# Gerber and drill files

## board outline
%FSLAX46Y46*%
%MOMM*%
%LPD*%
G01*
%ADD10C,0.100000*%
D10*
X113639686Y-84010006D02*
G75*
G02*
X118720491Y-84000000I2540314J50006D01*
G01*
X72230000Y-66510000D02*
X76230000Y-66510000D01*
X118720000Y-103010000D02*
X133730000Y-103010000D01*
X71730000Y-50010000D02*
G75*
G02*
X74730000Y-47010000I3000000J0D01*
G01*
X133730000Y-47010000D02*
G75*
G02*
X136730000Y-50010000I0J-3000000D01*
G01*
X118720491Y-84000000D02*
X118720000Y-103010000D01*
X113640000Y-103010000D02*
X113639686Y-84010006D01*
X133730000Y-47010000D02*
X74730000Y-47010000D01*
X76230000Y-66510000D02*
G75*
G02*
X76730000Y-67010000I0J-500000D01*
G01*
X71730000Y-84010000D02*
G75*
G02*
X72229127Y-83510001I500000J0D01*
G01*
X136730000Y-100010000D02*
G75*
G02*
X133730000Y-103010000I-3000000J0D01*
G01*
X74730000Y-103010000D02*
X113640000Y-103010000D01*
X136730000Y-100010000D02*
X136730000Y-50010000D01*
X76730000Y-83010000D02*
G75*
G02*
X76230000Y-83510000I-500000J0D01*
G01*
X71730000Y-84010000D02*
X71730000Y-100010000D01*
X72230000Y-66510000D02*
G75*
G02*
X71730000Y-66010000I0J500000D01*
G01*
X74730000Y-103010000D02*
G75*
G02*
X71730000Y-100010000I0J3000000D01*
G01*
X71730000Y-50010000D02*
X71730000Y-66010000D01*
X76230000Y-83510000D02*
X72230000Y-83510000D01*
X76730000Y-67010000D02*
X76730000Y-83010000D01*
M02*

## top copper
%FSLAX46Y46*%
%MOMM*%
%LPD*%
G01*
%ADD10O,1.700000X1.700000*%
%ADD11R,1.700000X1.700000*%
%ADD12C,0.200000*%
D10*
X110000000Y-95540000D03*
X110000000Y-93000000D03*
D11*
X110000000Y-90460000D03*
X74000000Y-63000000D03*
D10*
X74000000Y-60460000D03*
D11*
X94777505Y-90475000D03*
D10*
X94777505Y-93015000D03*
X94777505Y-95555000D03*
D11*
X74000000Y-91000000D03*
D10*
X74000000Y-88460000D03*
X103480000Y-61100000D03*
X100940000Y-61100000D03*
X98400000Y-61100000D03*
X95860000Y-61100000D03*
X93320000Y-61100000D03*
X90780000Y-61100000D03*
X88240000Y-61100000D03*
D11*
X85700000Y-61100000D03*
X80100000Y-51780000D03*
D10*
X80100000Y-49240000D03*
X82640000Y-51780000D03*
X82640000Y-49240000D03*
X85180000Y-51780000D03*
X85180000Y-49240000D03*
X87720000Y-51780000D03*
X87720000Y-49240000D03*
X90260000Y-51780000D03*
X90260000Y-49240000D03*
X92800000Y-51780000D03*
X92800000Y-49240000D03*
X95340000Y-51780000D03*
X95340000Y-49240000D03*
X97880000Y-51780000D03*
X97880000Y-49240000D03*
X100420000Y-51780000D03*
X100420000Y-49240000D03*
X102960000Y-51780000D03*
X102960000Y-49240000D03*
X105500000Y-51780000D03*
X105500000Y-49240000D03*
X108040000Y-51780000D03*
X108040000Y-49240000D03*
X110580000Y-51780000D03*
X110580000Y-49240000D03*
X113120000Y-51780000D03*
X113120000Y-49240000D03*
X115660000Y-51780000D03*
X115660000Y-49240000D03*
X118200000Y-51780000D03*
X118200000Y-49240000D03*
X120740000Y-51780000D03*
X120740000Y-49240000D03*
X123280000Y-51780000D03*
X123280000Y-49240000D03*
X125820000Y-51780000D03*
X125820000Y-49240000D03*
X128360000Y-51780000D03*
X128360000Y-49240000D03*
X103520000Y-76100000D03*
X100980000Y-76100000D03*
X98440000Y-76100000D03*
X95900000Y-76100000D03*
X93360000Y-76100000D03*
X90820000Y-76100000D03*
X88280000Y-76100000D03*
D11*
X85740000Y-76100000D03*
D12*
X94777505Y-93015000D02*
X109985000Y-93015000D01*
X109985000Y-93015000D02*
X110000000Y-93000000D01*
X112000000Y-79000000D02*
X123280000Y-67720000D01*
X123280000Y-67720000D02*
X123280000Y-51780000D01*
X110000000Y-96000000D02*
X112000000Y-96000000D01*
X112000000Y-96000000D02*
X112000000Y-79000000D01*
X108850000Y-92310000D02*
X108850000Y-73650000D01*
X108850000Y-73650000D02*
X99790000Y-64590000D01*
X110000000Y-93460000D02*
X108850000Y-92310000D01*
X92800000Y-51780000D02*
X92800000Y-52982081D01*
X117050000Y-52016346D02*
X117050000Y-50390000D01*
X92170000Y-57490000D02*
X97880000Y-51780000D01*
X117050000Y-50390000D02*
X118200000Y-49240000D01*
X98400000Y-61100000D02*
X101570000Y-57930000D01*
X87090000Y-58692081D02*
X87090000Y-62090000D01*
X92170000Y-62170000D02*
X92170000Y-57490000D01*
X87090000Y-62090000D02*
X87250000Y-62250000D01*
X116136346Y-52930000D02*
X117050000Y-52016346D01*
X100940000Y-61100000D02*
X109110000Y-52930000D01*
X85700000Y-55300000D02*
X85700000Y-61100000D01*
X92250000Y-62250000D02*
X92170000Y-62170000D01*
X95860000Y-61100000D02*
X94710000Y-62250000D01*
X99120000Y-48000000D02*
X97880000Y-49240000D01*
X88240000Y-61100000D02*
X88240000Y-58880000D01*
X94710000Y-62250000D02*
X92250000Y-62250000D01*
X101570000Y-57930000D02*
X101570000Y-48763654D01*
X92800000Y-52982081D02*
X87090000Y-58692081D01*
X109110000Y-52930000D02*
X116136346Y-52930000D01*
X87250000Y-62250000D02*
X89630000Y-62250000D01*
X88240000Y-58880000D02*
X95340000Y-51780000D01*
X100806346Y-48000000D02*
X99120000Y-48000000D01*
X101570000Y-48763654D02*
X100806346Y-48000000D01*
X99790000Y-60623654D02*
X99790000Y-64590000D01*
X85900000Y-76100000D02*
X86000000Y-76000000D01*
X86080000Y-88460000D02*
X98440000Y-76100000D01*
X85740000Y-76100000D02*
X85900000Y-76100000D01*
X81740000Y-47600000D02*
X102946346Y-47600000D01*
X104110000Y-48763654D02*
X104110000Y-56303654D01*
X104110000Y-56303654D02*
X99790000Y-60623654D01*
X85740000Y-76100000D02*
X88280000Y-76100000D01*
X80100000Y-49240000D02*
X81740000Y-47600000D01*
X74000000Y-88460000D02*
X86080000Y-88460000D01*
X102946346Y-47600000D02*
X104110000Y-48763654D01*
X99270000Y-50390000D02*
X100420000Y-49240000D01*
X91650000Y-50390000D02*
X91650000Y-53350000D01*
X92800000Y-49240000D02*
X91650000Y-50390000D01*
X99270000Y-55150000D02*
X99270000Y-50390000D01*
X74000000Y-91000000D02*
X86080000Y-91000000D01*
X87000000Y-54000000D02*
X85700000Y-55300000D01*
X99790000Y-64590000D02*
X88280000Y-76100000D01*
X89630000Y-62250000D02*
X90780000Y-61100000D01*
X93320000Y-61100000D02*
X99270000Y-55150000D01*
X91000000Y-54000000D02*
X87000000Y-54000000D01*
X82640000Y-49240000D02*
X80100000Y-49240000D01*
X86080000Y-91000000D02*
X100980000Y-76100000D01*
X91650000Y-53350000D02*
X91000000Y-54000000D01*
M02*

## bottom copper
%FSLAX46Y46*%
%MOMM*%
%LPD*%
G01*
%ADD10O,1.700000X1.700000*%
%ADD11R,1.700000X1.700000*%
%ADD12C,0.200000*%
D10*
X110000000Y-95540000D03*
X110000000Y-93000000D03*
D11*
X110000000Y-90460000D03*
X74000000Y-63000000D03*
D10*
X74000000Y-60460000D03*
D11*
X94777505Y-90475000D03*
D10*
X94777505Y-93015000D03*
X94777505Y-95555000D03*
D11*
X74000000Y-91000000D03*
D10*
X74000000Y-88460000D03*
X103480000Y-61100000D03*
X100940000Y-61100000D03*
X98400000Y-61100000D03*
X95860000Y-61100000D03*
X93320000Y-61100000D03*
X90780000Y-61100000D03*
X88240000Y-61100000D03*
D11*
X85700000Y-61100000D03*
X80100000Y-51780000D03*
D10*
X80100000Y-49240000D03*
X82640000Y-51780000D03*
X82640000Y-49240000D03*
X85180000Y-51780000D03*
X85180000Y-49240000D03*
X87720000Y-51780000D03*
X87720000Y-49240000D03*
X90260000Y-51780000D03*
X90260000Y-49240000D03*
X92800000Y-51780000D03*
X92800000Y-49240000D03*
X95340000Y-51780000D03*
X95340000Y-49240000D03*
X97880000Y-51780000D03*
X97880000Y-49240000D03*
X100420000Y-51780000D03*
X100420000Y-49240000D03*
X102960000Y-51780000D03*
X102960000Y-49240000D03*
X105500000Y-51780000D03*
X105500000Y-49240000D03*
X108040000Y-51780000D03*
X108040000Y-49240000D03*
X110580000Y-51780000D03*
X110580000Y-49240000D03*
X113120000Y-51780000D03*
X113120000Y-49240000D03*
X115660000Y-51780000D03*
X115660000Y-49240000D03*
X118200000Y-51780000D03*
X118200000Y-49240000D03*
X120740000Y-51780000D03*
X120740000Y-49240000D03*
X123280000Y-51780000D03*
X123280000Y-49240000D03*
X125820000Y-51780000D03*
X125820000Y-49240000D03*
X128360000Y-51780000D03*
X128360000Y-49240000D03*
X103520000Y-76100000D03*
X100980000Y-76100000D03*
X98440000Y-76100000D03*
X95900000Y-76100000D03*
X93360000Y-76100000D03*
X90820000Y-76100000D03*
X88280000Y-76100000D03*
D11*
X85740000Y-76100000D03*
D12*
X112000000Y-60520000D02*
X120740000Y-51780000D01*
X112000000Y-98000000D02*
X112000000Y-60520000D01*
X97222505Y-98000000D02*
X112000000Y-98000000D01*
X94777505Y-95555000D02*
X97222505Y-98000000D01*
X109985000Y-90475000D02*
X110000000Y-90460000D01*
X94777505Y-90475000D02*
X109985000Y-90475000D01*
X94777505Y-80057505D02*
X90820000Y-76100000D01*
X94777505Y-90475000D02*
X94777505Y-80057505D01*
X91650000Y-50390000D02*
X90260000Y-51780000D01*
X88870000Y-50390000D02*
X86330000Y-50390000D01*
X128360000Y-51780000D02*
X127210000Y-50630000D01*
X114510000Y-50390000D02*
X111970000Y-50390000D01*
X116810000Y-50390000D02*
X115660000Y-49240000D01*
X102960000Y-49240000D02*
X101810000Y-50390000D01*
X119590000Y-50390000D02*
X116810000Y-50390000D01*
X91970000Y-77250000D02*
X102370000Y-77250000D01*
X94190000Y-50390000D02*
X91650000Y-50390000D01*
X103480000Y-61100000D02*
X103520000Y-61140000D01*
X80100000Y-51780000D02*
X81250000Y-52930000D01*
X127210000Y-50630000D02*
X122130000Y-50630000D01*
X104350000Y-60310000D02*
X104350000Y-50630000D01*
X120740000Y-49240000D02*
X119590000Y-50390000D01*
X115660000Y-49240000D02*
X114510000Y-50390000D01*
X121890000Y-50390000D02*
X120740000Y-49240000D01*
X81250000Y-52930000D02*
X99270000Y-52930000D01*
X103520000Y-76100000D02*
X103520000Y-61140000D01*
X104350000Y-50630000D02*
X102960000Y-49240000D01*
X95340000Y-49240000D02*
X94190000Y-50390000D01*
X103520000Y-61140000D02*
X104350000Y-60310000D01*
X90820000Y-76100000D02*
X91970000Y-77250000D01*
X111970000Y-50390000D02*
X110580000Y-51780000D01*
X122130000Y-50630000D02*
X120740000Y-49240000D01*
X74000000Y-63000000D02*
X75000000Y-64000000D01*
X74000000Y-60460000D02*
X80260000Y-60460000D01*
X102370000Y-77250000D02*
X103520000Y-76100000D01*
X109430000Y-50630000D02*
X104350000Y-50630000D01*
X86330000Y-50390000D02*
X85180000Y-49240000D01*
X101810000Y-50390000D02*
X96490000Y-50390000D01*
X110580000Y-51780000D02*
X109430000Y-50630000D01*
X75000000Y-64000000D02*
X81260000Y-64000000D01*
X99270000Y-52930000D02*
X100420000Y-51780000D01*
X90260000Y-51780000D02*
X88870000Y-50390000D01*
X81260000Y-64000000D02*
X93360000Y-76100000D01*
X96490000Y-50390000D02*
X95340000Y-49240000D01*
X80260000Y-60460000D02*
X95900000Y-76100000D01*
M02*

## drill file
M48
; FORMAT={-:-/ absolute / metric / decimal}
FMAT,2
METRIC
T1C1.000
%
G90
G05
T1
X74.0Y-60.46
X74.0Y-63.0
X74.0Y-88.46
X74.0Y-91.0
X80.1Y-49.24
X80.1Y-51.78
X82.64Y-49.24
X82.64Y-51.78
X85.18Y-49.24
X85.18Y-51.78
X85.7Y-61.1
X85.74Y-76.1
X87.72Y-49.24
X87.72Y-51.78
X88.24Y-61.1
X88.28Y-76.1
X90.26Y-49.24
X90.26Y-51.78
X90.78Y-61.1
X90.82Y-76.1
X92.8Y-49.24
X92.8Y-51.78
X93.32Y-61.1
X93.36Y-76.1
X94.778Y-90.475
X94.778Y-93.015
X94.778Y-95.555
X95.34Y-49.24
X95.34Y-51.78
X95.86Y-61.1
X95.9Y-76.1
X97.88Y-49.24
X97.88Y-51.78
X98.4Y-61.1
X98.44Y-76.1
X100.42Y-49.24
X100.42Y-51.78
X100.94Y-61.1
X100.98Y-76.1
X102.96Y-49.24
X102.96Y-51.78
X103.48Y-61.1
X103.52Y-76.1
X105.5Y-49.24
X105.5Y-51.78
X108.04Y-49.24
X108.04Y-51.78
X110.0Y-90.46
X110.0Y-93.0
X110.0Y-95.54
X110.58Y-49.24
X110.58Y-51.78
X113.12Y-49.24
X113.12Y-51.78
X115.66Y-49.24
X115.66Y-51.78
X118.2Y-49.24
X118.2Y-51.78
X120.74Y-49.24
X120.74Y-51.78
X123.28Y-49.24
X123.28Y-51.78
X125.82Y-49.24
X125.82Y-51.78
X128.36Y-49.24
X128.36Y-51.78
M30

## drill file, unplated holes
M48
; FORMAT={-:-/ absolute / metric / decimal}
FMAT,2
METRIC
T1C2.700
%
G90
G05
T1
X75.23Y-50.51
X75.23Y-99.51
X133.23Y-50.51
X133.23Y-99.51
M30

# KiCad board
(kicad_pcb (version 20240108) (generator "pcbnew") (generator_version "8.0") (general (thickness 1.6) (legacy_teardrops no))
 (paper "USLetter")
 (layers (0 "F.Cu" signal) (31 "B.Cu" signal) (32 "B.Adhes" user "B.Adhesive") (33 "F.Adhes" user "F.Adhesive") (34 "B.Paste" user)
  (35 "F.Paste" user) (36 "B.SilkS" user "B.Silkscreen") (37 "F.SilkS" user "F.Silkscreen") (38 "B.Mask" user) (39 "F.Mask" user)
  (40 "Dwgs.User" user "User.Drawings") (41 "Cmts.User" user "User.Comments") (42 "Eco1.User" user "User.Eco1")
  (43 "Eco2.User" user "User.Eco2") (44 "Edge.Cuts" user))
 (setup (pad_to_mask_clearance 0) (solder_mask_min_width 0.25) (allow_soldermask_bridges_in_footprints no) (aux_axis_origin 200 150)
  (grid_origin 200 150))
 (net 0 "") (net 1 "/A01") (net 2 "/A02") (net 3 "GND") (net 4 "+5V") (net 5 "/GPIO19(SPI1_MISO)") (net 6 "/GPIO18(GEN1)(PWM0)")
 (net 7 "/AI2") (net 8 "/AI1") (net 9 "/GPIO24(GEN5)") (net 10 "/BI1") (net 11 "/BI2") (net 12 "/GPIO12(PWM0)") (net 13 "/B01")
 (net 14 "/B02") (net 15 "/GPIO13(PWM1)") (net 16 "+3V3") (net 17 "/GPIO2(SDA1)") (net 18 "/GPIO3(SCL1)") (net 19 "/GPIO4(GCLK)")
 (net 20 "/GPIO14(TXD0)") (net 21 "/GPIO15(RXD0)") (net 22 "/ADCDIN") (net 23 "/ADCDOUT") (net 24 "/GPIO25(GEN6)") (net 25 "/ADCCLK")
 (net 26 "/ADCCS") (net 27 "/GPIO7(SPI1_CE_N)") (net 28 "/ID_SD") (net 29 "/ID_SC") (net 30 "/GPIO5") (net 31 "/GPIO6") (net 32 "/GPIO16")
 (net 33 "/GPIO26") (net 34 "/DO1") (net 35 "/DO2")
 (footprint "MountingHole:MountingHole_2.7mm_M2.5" (layer "F.Cu") (at 133.23 99.51)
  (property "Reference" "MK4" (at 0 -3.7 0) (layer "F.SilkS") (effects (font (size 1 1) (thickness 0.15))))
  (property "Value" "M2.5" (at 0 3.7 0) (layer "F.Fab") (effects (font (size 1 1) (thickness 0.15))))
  (pad "" np_thru_hole circle (at 0 0) (size 2.7 2.7) (drill 2.7) (layers "*.Cu" "*.Mask")))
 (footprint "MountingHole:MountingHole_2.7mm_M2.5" (layer "F.Cu") (at 75.23 99.51)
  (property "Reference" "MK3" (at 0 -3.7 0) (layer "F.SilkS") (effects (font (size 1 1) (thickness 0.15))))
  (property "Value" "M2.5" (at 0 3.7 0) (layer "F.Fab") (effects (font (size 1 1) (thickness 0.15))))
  (pad "" np_thru_hole circle (at 0 0) (size 2.7 2.7) (drill 2.7) (layers "*.Cu" "*.Mask")))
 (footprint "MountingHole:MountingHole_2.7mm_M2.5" (layer "F.Cu") (at 75.23 50.51 180)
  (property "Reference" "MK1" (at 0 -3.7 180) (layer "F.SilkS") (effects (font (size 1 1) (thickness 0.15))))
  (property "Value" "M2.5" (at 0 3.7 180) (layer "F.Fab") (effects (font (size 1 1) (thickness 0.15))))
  (pad "" np_thru_hole circle (at 0 0 180) (size 2.7 2.7) (drill 2.7) (layers "*.Cu" "*.Mask")))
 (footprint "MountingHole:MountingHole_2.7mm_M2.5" (layer "F.Cu") (at 133.23 50.51 180)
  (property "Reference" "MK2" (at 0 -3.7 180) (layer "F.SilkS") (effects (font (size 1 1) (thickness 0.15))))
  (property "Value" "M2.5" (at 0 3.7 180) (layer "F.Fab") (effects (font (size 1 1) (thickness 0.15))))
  (pad "" np_thru_hole circle (at 0 0 180) (size 2.7 2.7) (drill 2.7) (layers "*.Cu" "*.Mask")))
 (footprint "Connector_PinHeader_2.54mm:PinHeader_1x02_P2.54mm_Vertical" (layer "F.Cu") (at 74 63 180)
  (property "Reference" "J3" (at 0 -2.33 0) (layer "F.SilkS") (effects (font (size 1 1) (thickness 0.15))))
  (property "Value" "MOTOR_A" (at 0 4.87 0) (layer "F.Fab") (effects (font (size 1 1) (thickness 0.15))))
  (pad "1" thru_hole rect (at 0 0 180) (size 1.7 1.7) (drill 1) (layers "*.Cu" "*.Mask") (remove_unused_layers no) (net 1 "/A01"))
  (pad "2" thru_hole oval (at 0 2.54 180) (size 1.7 1.7) (drill 1) (layers "*.Cu" "*.Mask") (remove_unused_layers no) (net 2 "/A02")))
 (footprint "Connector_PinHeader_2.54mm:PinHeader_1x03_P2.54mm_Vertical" (layer "F.Cu") (at 110 90.46)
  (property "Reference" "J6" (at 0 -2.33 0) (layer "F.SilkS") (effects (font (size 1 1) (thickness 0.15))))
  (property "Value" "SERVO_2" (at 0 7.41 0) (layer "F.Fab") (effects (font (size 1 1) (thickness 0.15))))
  (pad "1" thru_hole rect (at 0 0) (size 1.7 1.7) (drill 1) (layers "*.Cu" "*.Mask") (remove_unused_layers no) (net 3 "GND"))
  (pad "2" thru_hole oval (at 0 2.54) (size 1.7 1.7) (drill 1) (layers "*.Cu" "*.Mask") (remove_unused_layers no) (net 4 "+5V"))
  (pad "3" thru_hole oval (at 0 5.08) (size 1.7 1.7) (drill 1) (layers "*.Cu" "*.Mask") (remove_unused_layers no)
   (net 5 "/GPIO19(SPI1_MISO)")))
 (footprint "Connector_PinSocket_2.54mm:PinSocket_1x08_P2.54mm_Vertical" (layer "F.Cu") (at 85.7 61.1 90)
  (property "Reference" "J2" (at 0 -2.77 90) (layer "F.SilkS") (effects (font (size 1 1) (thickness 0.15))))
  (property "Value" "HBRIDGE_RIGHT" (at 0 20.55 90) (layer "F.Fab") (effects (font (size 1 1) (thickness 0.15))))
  (pad "1" thru_hole rect (at 0 0 90) (size 1.7 1.7) (drill 1) (layers "*.Cu" "*.Mask") (remove_unused_layers no)
   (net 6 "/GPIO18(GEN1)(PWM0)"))
  (pad "2" thru_hole oval (at 0 2.54 90) (size 1.7 1.7) (drill 1) (layers "*.Cu" "*.Mask") (remove_unused_layers no) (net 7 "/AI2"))
  (pad "3" thru_hole oval (at 0 5.08 90) (size 1.7 1.7) (drill 1) (layers "*.Cu" "*.Mask") (remove_unused_layers no) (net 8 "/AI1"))
  (pad "4" thru_hole oval (at 0 7.62 90) (size 1.7 1.7) (drill 1) (layers "*.Cu" "*.Mask") (remove_unused_layers no) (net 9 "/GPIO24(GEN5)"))
  (pad "5" thru_hole oval (at 0 10.16 90) (size 1.7 1.7) (drill 1) (layers "*.Cu" "*.Mask") (remove_unused_layers no) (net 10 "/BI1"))
  (pad "6" thru_hole oval (at 0 12.7 90) (size 1.7 1.7) (drill 1) (layers "*.Cu" "*.Mask") (remove_unused_layers no) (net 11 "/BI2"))
  (pad "7" thru_hole oval (at 0 15.24 90) (size 1.7 1.7) (drill 1) (layers "*.Cu" "*.Mask") (remove_unused_layers no)
   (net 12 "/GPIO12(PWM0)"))
  (pad "8" thru_hole oval (at 0 17.78 90) (size 1.7 1.7) (drill 1) (layers "*.Cu" "*.Mask") (remove_unused_layers no) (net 3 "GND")))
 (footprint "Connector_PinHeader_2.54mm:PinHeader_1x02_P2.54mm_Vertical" (layer "F.Cu") (at 74 91 180)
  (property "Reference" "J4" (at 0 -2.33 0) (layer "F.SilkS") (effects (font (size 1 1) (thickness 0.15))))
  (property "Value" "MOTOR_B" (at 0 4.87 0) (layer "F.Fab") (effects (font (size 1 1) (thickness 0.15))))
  (pad "1" thru_hole rect (at 0 0 180) (size 1.7 1.7) (drill 1) (layers "*.Cu" "*.Mask") (remove_unused_layers no) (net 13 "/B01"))
  (pad "2" thru_hole oval (at 0 2.54 180) (size 1.7 1.7) (drill 1) (layers "*.Cu" "*.Mask") (remove_unused_layers no) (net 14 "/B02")))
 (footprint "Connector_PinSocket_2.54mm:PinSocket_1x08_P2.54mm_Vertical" (layer "F.Cu") (at 85.74 76.1 90)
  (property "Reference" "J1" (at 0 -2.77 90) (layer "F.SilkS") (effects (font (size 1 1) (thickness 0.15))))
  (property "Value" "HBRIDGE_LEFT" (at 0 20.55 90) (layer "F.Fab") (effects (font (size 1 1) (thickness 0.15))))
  (pad "1" thru_hole rect (at 0 0 90) (size 1.7 1.7) (drill 1) (layers "*.Cu" "*.Mask") (remove_unused_layers no) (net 4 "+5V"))
  (pad "2" thru_hole oval (at 0 2.54 90) (size 1.7 1.7) (drill 1) (layers "*.Cu" "*.Mask") (remove_unused_layers no) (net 4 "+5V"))
  (pad "3" thru_hole oval (at 0 5.08 90) (size 1.7 1.7) (drill 1) (layers "*.Cu" "*.Mask") (remove_unused_layers no) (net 3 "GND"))
  (pad "4" thru_hole oval (at 0 7.62 90) (size 1.7 1.7) (drill 1) (layers "*.Cu" "*.Mask") (remove_unused_layers no) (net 1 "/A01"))
  (pad "5" thru_hole oval (at 0 10.16 90) (size 1.7 1.7) (drill 1) (layers "*.Cu" "*.Mask") (remove_unused_layers no) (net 2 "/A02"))
  (pad "6" thru_hole oval (at 0 12.7 90) (size 1.7 1.7) (drill 1) (layers "*.Cu" "*.Mask") (remove_unused_layers no) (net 14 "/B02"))
  (pad "7" thru_hole oval (at 0 15.24 90) (size 1.7 1.7) (drill 1) (layers "*.Cu" "*.Mask") (remove_unused_layers no) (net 13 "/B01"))
  (pad "8" thru_hole oval (at 0 17.78 90) (size 1.7 1.7) (drill 1) (layers "*.Cu" "*.Mask") (remove_unused_layers no) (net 3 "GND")))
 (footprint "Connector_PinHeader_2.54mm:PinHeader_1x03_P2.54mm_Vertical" (layer "F.Cu") (at 94.777505 90.475)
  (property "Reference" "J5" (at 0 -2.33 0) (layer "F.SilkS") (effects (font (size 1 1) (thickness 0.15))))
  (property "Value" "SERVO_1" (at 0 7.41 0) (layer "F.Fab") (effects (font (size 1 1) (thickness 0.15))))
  (pad "1" thru_hole rect (at 0 0) (size 1.7 1.7) (drill 1) (layers "*.Cu" "*.Mask") (remove_unused_layers no) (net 3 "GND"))
  (pad "2" thru_hole oval (at 0 2.54) (size 1.7 1.7) (drill 1) (layers "*.Cu" "*.Mask") (remove_unused_layers no) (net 4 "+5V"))
  (pad "3" thru_hole oval (at 0 5.08) (size 1.7 1.7) (drill 1) (layers "*.Cu" "*.Mask") (remove_unused_layers no) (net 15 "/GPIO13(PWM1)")))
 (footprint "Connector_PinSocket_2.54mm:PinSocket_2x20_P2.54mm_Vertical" (layer "B.Cu") (at 80.1 51.78 -90)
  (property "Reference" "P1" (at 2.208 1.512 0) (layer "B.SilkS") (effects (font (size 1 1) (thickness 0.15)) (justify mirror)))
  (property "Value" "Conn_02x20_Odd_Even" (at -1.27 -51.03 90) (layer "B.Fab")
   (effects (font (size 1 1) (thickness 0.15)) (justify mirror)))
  (pad "1" thru_hole rect (at 0 0 270) (size 1.7 1.7) (drill 1) (layers "*.Cu" "*.Mask") (remove_unused_layers no) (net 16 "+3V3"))
  (pad "2" thru_hole oval (at -2.54 0 270) (size 1.7 1.7) (drill 1) (layers "*.Cu" "*.Mask") (remove_unused_layers no) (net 4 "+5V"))
  (pad "3" thru_hole oval (at 0 -2.54 270) (size 1.7 1.7) (drill 1) (layers "*.Cu" "*.Mask") (remove_unused_layers no)
   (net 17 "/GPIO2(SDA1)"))
  (pad "4" thru_hole oval (at -2.54 -2.54 270) (size 1.7 1.7) (drill 1) (layers "*.Cu" "*.Mask") (remove_unused_layers no) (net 4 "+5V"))
  (pad "5" thru_hole oval (at 0 -5.08 270) (size 1.7 1.7) (drill 1) (layers "*.Cu" "*.Mask") (remove_unused_layers no)
   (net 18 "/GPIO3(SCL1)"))
  (pad "6" thru_hole oval (at -2.54 -5.08 270) (size 1.7 1.7) (drill 1) (layers "*.Cu" "*.Mask") (remove_unused_layers no) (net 3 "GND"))
  (pad "7" thru_hole oval (at 0 -7.62 270) (size 1.7 1.7) (drill 1) (layers "*.Cu" "*.Mask") (remove_unused_layers no)
   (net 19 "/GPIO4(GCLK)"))
  (pad "8" thru_hole oval (at -2.54 -7.62 270) (size 1.7 1.7) (drill 1) (layers "*.Cu" "*.Mask") (remove_unused_layers no)
   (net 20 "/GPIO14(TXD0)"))
  (pad "9" thru_hole oval (at 0 -10.16 270) (size 1.7 1.7) (drill 1) (layers "*.Cu" "*.Mask") (remove_unused_layers no) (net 3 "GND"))
  (pad "10" thru_hole oval (at -2.54 -10.16 270) (size 1.7 1.7) (drill 1) (layers "*.Cu" "*.Mask") (remove_unused_layers no)
   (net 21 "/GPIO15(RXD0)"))
  (pad "11" thru_hole oval (at 0 -12.7 270) (size 1.7 1.7) (drill 1) (layers "*.Cu" "*.Mask") (remove_unused_layers no) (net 8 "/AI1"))
  (pad "12" thru_hole oval (at -2.54 -12.7 270) (size 1.7 1.7) (drill 1) (layers "*.Cu" "*.Mask") (remove_unused_layers no)
   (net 6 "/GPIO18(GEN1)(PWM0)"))
  (pad "13" thru_hole oval (at 0 -15.24 270) (size 1.7 1.7) (drill 1) (layers "*.Cu" "*.Mask") (remove_unused_layers no) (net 7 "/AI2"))
  (pad "14" thru_hole oval (at -2.54 -15.24 270) (size 1.7 1.7) (drill 1) (layers "*.Cu" "*.Mask") (remove_unused_layers no) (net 3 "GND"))
  (pad "15" thru_hole oval (at 0 -17.78 270) (size 1.7 1.7) (drill 1) (layers "*.Cu" "*.Mask") (remove_unused_layers no) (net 10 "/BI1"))
  (pad "16" thru_hole oval (at -2.54 -17.78 270) (size 1.7 1.7) (drill 1) (layers "*.Cu" "*.Mask") (remove_unused_layers no) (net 11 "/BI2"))
  (pad "17" thru_hole oval (at 0 -20.32 270) (size 1.7 1.7) (drill 1) (layers "*.Cu" "*.Mask") (remove_unused_layers no) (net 16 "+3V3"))
  (pad "18" thru_hole oval (at -2.54 -20.32 270) (size 1.7 1.7) (drill 1) (layers "*.Cu" "*.Mask") (remove_unused_layers no)
   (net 9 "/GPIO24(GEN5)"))
  (pad "19" thru_hole oval (at 0 -22.86 270) (size 1.7 1.7) (drill 1) (layers "*.Cu" "*.Mask") (remove_unused_layers no) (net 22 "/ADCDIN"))
  (pad "20" thru_hole oval (at -2.54 -22.86 270) (size 1.7 1.7) (drill 1) (layers "*.Cu" "*.Mask") (remove_unused_layers no) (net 3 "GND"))
  (pad "21" thru_hole oval (at 0 -25.4 270) (size 1.7 1.7) (drill 1) (layers "*.Cu" "*.Mask") (remove_unused_layers no) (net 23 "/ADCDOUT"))
  (pad "22" thru_hole oval (at -2.54 -25.4 270) (size 1.7 1.7) (drill 1) (layers "*.Cu" "*.Mask") (remove_unused_layers no)
   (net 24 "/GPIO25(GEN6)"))
  (pad "23" thru_hole oval (at 0 -27.94 270) (size 1.7 1.7) (drill 1) (layers "*.Cu" "*.Mask") (remove_unused_layers no) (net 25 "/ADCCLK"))
  (pad "24" thru_hole oval (at -2.54 -27.94 270) (size 1.7 1.7) (drill 1) (layers "*.Cu" "*.Mask") (remove_unused_layers no)
   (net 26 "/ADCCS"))
  (pad "25" thru_hole oval (at 0 -30.48 270) (size 1.7 1.7) (drill 1) (layers "*.Cu" "*.Mask") (remove_unused_layers no) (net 3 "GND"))
  (pad "26" thru_hole oval (at -2.54 -30.48 270) (size 1.7 1.7) (drill 1) (layers "*.Cu" "*.Mask") (remove_unused_layers no)
   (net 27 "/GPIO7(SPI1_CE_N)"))
  (pad "27" thru_hole oval (at 0 -33.02 270) (size 1.7 1.7) (drill 1) (layers "*.Cu" "*.Mask") (remove_unused_layers no) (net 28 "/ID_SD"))
  (pad "28" thru_hole oval (at -2.54 -33.02 270) (size 1.7 1.7) (drill 1) (layers "*.Cu" "*.Mask") (remove_unused_layers no)
   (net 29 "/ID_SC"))
  (pad "29" thru_hole oval (at 0 -35.56 270) (size 1.7 1.7) (drill 1) (layers "*.Cu" "*.Mask") (remove_unused_layers no) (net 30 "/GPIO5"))
  (pad "30" thru_hole oval (at -2.54 -35.56 270) (size 1.7 1.7) (drill 1) (layers "*.Cu" "*.Mask") (remove_unused_layers no) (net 3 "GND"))
  (pad "31" thru_hole oval (at 0 -38.1 270) (size 1.7 1.7) (drill 1) (layers "*.Cu" "*.Mask") (remove_unused_layers no) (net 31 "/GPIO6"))
  (pad "32" thru_hole oval (at -2.54 -38.1 270) (size 1.7 1.7) (drill 1) (layers "*.Cu" "*.Mask") (remove_unused_layers no)
   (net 12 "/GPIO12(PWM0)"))
  (pad "33" thru_hole oval (at 0 -40.64 270) (size 1.7 1.7) (drill 1) (layers "*.Cu" "*.Mask") (remove_unused_layers no)
   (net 15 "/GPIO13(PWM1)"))
  (pad "34" thru_hole oval (at -2.54 -40.64 270) (size 1.7 1.7) (drill 1) (layers "*.Cu" "*.Mask") (remove_unused_layers no) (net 3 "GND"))
  (pad "35" thru_hole oval (at 0 -43.18 270) (size 1.7 1.7) (drill 1) (layers "*.Cu" "*.Mask") (remove_unused_layers no)
   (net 5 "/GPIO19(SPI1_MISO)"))
  (pad "36" thru_hole oval (at -2.54 -43.18 270) (size 1.7 1.7) (drill 1) (layers "*.Cu" "*.Mask") (remove_unused_layers no)
   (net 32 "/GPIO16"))
  (pad "37" thru_hole oval (at 0 -45.72 270) (size 1.7 1.7) (drill 1) (layers "*.Cu" "*.Mask") (remove_unused_layers no) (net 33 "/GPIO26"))
  (pad "38" thru_hole oval (at -2.54 -45.72 270) (size 1.7 1.7) (drill 1) (layers "*.Cu" "*.Mask") (remove_unused_layers no) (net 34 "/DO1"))
  (pad "39" thru_hole oval (at 0 -48.26 270) (size 1.7 1.7) (drill 1) (layers "*.Cu" "*.Mask") (remove_unused_layers no) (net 3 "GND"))
  (pad "40" thru_hole oval (at -2.54 -48.26 270) (size 1.7 1.7) (drill 1) (layers "*.Cu" "*.Mask") (remove_unused_layers no) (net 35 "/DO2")))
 (gr_line (start 71.73 84.01) (end 71.73 100.01) (stroke (width 0.1) (type solid)) (layer "Edge.Cuts"))
 (gr_line (start 136.73 100.01) (end 136.73 50.01) (stroke (width 0.1) (type solid)) (layer "Edge.Cuts"))
 (gr_line (start 74.73 103.01) (end 113.64 103.01) (stroke (width 0.1) (type solid)) (layer "Edge.Cuts"))
 (gr_arc (start 76.73 83.01) (mid 76.583553 83.363553) (end 76.23 83.51) (stroke (width 0.1) (type solid)) (layer "Edge.Cuts"))
 (gr_line (start 76.23 83.51) (end 72.23 83.51) (stroke (width 0.1) (type solid)) (layer "Edge.Cuts"))
 (gr_arc (start 113.639686 84.010006) (mid 116.174996 81.419199) (end 118.720491 84) (locked yes) (stroke (width 0.1) (type solid))
  (layer "Edge.Cuts"))
 (gr_arc (start 133.73 47.01) (mid 135.85132 47.88868) (end 136.73 50.01) (stroke (width 0.1) (type solid)) (layer "Edge.Cuts"))
 (gr_arc (start 72.23 66.51) (mid 71.876447 66.363553) (end 71.73 66.01) (stroke (width 0.1) (type solid)) (layer "Edge.Cuts"))
 (gr_arc (start 136.73 100.01) (mid 135.85132 102.13132) (end 133.73 103.01) (stroke (width 0.1) (type solid)) (layer "Edge.Cuts"))
 (gr_arc (start 71.73 84.01) (mid 71.876138 83.656755) (end 72.229127 83.510001) (stroke (width 0.1) (type solid)) (layer "Edge.Cuts"))
 (gr_arc (start 74.73 103.01) (mid 72.60868 102.13132) (end 71.73 100.01) (stroke (width 0.1) (type solid)) (layer "Edge.Cuts"))
 (gr_arc (start 76.23 66.51) (mid 76.583553 66.656447) (end 76.73 67.01) (stroke (width 0.1) (type solid)) (layer "Edge.Cuts"))
 (gr_arc (start 71.73 50.01) (mid 72.60868 47.88868) (end 74.73 47.01) (stroke (width 0.1) (type solid)) (layer "Edge.Cuts"))
 (gr_line (start 133.73 47.01) (end 74.73 47.01) (stroke (width 0.1) (type solid)) (layer "Edge.Cuts"))
 (gr_line (start 72.23 66.51) (end 76.23 66.51) (stroke (width 0.1) (type solid)) (layer "Edge.Cuts"))
 (gr_line (start 71.73 50.01) (end 71.73 66.01) (stroke (width 0.1) (type solid)) (layer "Edge.Cuts"))
 (gr_line (start 76.73 67.01) (end 76.73 83.01) (stroke (width 0.1) (type solid)) (layer "Edge.Cuts"))
 (gr_line (start 113.64 103.01) (end 113.639686 84.010006) (stroke (width 0.1) (type default)) (layer "Edge.Cuts"))
 (gr_line (start 118.72 103.01) (end 133.73 103.01) (stroke (width 0.1) (type default)) (layer "Edge.Cuts"))
 (gr_line (start 118.720491 84) (end 118.72 103.01) (stroke (width 0.1) (type default)) (layer "Edge.Cuts"))
 (segment (start 81.25 52.93) (end 99.27 52.93) (width 0.2) (layer "B.Cu") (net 16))
 (segment (start 99.27 52.93) (end 100.42 51.78) (width 0.2) (layer "B.Cu") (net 16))
 (segment (start 80.1 51.78) (end 81.25 52.93) (width 0.2) (layer "B.Cu") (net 16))
 (segment (start 108.85 73.65) (end 99.79 64.59) (width 0.2) (layer "F.Cu") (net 4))
 (segment (start 82.64 49.24) (end 80.1 49.24) (width 0.2) (layer "F.Cu") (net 4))
 (segment (start 85.74 76.1) (end 85.9 76.1) (width 0.2) (layer "F.Cu") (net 4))
 (segment (start 108.85 92.31) (end 108.85 73.65) (width 0.2) (layer "F.Cu") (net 4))
 (segment (start 80.1 49.24) (end 81.74 47.6) (width 0.2) (layer "F.Cu") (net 4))
 (segment (start 99.79 64.59) (end 88.28 76.1) (width 0.2) (layer "F.Cu") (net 4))
 (segment (start 94.777505 93.015) (end 109.985 93.015) (width 0.2) (layer "F.Cu") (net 4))
 (segment (start 110 93.46) (end 108.85 92.31) (width 0.2) (layer "F.Cu") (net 4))
 (segment (start 102.946346 47.6) (end 104.11 48.763654) (width 0.2) (layer "F.Cu") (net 4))
 (segment (start 99.79 60.623654) (end 99.79 64.59) (width 0.2) (layer "F.Cu") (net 4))
 (segment (start 85.74 76.1) (end 88.28 76.1) (width 0.2) (layer "F.Cu") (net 4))
 (segment (start 81.74 47.6) (end 102.946346 47.6) (width 0.2) (layer "F.Cu") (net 4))
 (segment (start 104.11 56.303654) (end 99.79 60.623654) (width 0.2) (layer "F.Cu") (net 4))
 (segment (start 109.985 93.015) (end 110 93) (width 0.2) (layer "F.Cu") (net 4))
 (segment (start 104.11 48.763654) (end 104.11 56.303654) (width 0.2) (layer "F.Cu") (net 4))
 (segment (start 85.9 76.1) (end 86 76) (width 0.2) (layer "F.Cu") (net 4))
 (segment (start 114.51 50.39) (end 111.97 50.39) (width 0.2) (layer "B.Cu") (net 3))
 (segment (start 103.48 61.1) (end 103.52 61.14) (width 0.2) (layer "B.Cu") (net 3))
 (segment (start 128.36 51.78) (end 127.21 50.63) (width 0.2) (layer "B.Cu") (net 3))
 (segment (start 88.87 50.39) (end 86.33 50.39) (width 0.2) (layer "B.Cu") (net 3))
 (segment (start 122.13 50.63) (end 120.74 49.24) (width 0.2) (layer "B.Cu") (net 3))
 (segment (start 90.82 76.1) (end 91.97 77.25) (width 0.2) (layer "B.Cu") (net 3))
 (segment (start 90.26 51.78) (end 88.87 50.39) (width 0.2) (layer "B.Cu") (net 3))
 (segment (start 103.52 61.14) (end 104.35 60.31) (width 0.2) (layer "B.Cu") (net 3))
 (segment (start 109.985 90.475) (end 110 90.46) (width 0.2) (layer "B.Cu") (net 3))
 (segment (start 120.74 49.24) (end 119.59 50.39) (width 0.2) (layer "B.Cu") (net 3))
 (segment (start 95.34 49.24) (end 94.19 50.39) (width 0.2) (layer "B.Cu") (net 3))
 (segment (start 119.59 50.39) (end 116.81 50.39) (width 0.2) (layer "B.Cu") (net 3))
 (segment (start 102.37 77.25) (end 103.52 76.1) (width 0.2) (layer "B.Cu") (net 3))
 (segment (start 96.49 50.39) (end 95.34 49.24) (width 0.2) (layer "B.Cu") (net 3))
 (segment (start 104.35 60.31) (end 104.35 50.63) (width 0.2) (layer "B.Cu") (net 3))
 (segment (start 94.777505 90.475) (end 109.985 90.475) (width 0.2) (layer "B.Cu") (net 3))
 (segment (start 86.33 50.39) (end 85.18 49.24) (width 0.2) (layer "B.Cu") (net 3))
 (segment (start 111.97 50.39) (end 110.58 51.78) (width 0.2) (layer "B.Cu") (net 3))
 (segment (start 115.66 49.24) (end 114.51 50.39) (width 0.2) (layer "B.Cu") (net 3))
 (segment (start 104.35 50.63) (end 102.96 49.24) (width 0.2) (layer "B.Cu") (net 3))
 (segment (start 116.81 50.39) (end 115.66 49.24) (width 0.2) (layer "B.Cu") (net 3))
 (segment (start 94.777505 90.475) (end 94.777505 80.057505) (width 0.2) (layer "B.Cu") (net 3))
 (segment (start 103.52 76.1) (end 103.52 61.14) (width 0.2) (layer "B.Cu") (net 3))
 (segment (start 121.89 50.39) (end 120.74 49.24) (width 0.2) (layer "B.Cu") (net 3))
 (segment (start 109.43 50.63) (end 104.35 50.63) (width 0.2) (layer "B.Cu") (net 3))
 (segment (start 102.96 49.24) (end 101.81 50.39) (width 0.2) (layer "B.Cu") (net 3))
 (segment (start 94.19 50.39) (end 91.65 50.39) (width 0.2) (layer "B.Cu") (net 3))
 (segment (start 94.777505 80.057505) (end 90.82 76.1) (width 0.2) (layer "B.Cu") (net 3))
 (segment (start 110.58 51.78) (end 109.43 50.63) (width 0.2) (layer "B.Cu") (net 3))
 (segment (start 91.65 50.39) (end 90.26 51.78) (width 0.2) (layer "B.Cu") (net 3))
 (segment (start 101.81 50.39) (end 96.49 50.39) (width 0.2) (layer "B.Cu") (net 3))
 (segment (start 127.21 50.63) (end 122.13 50.63) (width 0.2) (layer "B.Cu") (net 3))
 (segment (start 91.97 77.25) (end 102.37 77.25) (width 0.2) (layer "B.Cu") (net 3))
 (segment (start 86.08 88.46) (end 98.44 76.1) (width 0.2) (layer "F.Cu") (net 14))
 (segment (start 74 88.46) (end 86.08 88.46) (width 0.2) (layer "F.Cu") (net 14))
 (segment (start 74 60.46) (end 80.26 60.46) (width 0.2) (layer "B.Cu") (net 2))
 (segment (start 80.26 60.46) (end 95.9 76.1) (width 0.2) (layer "B.Cu") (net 2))
 (segment (start 81.26 64) (end 93.36 76.1) (width 0.2) (layer "B.Cu") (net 1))
 (segment (start 74 63) (end 75 64) (width 0.2) (layer "B.Cu") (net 1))
 (segment (start 75 64) (end 81.26 64) (width 0.2) (layer "B.Cu") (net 1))
 (segment (start 86.08 91) (end 100.98 76.1) (width 0.2) (layer "F.Cu") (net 13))
 (segment (start 74 91) (end 86.08 91) (width 0.2) (layer "F.Cu") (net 13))
 (segment (start 99.27 55.15) (end 99.27 50.39) (width 0.2) (layer "F.Cu") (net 9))
 (segment (start 93.32 61.1) (end 99.27 55.15) (width 0.2) (layer "F.Cu") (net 9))
 (segment (start 99.27 50.39) (end 100.42 49.24) (width 0.2) (layer "F.Cu") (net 9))
 (segment (start 91.65 53.35) (end 91 54) (width 0.2) (layer "F.Cu") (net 6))
 (segment (start 87 54) (end 85.7 55.3) (width 0.2) (layer "F.Cu") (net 6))
 (segment (start 91 54) (end 87 54) (width 0.2) (layer "F.Cu") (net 6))
 (segment (start 92.8 49.24) (end 91.65 50.39) (width 0.2) (layer "F.Cu") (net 6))
 (segment (start 91.65 50.39) (end 91.65 53.35) (width 0.2) (layer "F.Cu") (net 6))
 (segment (start 85.7 55.3) (end 85.7 61.1) (width 0.2) (layer "F.Cu") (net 6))
 (segment (start 116.136346 52.93) (end 117.05 52.016346) (width 0.2) (layer "F.Cu") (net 12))
 (segment (start 109.11 52.93) (end 116.136346 52.93) (width 0.2) (layer "F.Cu") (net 12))
 (segment (start 117.05 52.016346) (end 117.05 50.39) (width 0.2) (layer "F.Cu") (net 12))
 (segment (start 100.94 61.1) (end 109.11 52.93) (width 0.2) (layer "F.Cu") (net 12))
 (segment (start 117.05 50.39) (end 118.2 49.24) (width 0.2) (layer "F.Cu") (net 12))
 (segment (start 112 60.52) (end 120.74 51.78) (width 0.2) (layer "B.Cu") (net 15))
 (segment (start 97.222505 98) (end 112 98) (width 0.2) (layer "B.Cu") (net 15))
 (segment (start 112 98) (end 112 60.52) (width 0.2) (layer "B.Cu") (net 15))
 (segment (start 94.777505 95.555) (end 97.222505 98) (width 0.2) (layer "B.Cu") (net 15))
 (segment (start 112 96) (end 112 79) (width 0.2) (layer "F.Cu") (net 5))
 (segment (start 112 79) (end 123.28 67.72) (width 0.2) (layer "F.Cu") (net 5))
 (segment (start 123.28 67.72) (end 123.28 51.78) (width 0.2) (layer "F.Cu") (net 5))
 (segment (start 110 96) (end 112 96) (width 0.2) (layer "F.Cu") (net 5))
 (segment (start 87.09 58.692081) (end 87.09 62.09) (width 0.2) (layer "F.Cu") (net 8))
 (segment (start 87.25 62.25) (end 89.63 62.25) (width 0.2) (layer "F.Cu") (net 8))
 (segment (start 87.09 62.09) (end 87.25 62.25) (width 0.2) (layer "F.Cu") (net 8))
 (segment (start 92.8 52.982081) (end 87.09 58.692081) (width 0.2) (layer "F.Cu") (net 8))
 (segment (start 92.8 51.78) (end 92.8 52.982081) (width 0.2) (layer "F.Cu") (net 8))
 (segment (start 89.63 62.25) (end 90.78 61.1) (width 0.2) (layer "F.Cu") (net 8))
 (segment (start 98.4 61.1) (end 101.57 57.93) (width 0.2) (layer "F.Cu") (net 11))
 (segment (start 99.12 48) (end 97.88 49.24) (width 0.2) (layer "F.Cu") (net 11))
 (segment (start 100.806346 48) (end 99.12 48) (width 0.2) (layer "F.Cu") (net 11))
 (segment (start 101.57 57.93) (end 101.57 48.763654) (width 0.2) (layer "F.Cu") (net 11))
 (segment (start 101.57 48.763654) (end 100.806346 48) (width 0.2) (layer "F.Cu") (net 11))
 (segment (start 92.17 62.17) (end 92.17 57.49) (width 0.2) (layer "F.Cu") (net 10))
 (segment (start 92.25 62.25) (end 92.17 62.17) (width 0.2) (layer "F.Cu") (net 10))
 (segment (start 92.17 57.49) (end 97.88 51.78) (width 0.2) (layer "F.Cu") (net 10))
 (segment (start 94.71 62.25) (end 92.25 62.25) (width 0.2) (layer "F.Cu") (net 10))
 (segment (start 95.86 61.1) (end 94.71 62.25) (width 0.2) (layer "F.Cu") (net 10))
 (segment (start 88.24 58.88) (end 95.34 51.78) (width 0.2) (layer "F.Cu") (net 7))
 (segment (start 88.24 61.1) (end 88.24 58.88) (width 0.2) (layer "F.Cu") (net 7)))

